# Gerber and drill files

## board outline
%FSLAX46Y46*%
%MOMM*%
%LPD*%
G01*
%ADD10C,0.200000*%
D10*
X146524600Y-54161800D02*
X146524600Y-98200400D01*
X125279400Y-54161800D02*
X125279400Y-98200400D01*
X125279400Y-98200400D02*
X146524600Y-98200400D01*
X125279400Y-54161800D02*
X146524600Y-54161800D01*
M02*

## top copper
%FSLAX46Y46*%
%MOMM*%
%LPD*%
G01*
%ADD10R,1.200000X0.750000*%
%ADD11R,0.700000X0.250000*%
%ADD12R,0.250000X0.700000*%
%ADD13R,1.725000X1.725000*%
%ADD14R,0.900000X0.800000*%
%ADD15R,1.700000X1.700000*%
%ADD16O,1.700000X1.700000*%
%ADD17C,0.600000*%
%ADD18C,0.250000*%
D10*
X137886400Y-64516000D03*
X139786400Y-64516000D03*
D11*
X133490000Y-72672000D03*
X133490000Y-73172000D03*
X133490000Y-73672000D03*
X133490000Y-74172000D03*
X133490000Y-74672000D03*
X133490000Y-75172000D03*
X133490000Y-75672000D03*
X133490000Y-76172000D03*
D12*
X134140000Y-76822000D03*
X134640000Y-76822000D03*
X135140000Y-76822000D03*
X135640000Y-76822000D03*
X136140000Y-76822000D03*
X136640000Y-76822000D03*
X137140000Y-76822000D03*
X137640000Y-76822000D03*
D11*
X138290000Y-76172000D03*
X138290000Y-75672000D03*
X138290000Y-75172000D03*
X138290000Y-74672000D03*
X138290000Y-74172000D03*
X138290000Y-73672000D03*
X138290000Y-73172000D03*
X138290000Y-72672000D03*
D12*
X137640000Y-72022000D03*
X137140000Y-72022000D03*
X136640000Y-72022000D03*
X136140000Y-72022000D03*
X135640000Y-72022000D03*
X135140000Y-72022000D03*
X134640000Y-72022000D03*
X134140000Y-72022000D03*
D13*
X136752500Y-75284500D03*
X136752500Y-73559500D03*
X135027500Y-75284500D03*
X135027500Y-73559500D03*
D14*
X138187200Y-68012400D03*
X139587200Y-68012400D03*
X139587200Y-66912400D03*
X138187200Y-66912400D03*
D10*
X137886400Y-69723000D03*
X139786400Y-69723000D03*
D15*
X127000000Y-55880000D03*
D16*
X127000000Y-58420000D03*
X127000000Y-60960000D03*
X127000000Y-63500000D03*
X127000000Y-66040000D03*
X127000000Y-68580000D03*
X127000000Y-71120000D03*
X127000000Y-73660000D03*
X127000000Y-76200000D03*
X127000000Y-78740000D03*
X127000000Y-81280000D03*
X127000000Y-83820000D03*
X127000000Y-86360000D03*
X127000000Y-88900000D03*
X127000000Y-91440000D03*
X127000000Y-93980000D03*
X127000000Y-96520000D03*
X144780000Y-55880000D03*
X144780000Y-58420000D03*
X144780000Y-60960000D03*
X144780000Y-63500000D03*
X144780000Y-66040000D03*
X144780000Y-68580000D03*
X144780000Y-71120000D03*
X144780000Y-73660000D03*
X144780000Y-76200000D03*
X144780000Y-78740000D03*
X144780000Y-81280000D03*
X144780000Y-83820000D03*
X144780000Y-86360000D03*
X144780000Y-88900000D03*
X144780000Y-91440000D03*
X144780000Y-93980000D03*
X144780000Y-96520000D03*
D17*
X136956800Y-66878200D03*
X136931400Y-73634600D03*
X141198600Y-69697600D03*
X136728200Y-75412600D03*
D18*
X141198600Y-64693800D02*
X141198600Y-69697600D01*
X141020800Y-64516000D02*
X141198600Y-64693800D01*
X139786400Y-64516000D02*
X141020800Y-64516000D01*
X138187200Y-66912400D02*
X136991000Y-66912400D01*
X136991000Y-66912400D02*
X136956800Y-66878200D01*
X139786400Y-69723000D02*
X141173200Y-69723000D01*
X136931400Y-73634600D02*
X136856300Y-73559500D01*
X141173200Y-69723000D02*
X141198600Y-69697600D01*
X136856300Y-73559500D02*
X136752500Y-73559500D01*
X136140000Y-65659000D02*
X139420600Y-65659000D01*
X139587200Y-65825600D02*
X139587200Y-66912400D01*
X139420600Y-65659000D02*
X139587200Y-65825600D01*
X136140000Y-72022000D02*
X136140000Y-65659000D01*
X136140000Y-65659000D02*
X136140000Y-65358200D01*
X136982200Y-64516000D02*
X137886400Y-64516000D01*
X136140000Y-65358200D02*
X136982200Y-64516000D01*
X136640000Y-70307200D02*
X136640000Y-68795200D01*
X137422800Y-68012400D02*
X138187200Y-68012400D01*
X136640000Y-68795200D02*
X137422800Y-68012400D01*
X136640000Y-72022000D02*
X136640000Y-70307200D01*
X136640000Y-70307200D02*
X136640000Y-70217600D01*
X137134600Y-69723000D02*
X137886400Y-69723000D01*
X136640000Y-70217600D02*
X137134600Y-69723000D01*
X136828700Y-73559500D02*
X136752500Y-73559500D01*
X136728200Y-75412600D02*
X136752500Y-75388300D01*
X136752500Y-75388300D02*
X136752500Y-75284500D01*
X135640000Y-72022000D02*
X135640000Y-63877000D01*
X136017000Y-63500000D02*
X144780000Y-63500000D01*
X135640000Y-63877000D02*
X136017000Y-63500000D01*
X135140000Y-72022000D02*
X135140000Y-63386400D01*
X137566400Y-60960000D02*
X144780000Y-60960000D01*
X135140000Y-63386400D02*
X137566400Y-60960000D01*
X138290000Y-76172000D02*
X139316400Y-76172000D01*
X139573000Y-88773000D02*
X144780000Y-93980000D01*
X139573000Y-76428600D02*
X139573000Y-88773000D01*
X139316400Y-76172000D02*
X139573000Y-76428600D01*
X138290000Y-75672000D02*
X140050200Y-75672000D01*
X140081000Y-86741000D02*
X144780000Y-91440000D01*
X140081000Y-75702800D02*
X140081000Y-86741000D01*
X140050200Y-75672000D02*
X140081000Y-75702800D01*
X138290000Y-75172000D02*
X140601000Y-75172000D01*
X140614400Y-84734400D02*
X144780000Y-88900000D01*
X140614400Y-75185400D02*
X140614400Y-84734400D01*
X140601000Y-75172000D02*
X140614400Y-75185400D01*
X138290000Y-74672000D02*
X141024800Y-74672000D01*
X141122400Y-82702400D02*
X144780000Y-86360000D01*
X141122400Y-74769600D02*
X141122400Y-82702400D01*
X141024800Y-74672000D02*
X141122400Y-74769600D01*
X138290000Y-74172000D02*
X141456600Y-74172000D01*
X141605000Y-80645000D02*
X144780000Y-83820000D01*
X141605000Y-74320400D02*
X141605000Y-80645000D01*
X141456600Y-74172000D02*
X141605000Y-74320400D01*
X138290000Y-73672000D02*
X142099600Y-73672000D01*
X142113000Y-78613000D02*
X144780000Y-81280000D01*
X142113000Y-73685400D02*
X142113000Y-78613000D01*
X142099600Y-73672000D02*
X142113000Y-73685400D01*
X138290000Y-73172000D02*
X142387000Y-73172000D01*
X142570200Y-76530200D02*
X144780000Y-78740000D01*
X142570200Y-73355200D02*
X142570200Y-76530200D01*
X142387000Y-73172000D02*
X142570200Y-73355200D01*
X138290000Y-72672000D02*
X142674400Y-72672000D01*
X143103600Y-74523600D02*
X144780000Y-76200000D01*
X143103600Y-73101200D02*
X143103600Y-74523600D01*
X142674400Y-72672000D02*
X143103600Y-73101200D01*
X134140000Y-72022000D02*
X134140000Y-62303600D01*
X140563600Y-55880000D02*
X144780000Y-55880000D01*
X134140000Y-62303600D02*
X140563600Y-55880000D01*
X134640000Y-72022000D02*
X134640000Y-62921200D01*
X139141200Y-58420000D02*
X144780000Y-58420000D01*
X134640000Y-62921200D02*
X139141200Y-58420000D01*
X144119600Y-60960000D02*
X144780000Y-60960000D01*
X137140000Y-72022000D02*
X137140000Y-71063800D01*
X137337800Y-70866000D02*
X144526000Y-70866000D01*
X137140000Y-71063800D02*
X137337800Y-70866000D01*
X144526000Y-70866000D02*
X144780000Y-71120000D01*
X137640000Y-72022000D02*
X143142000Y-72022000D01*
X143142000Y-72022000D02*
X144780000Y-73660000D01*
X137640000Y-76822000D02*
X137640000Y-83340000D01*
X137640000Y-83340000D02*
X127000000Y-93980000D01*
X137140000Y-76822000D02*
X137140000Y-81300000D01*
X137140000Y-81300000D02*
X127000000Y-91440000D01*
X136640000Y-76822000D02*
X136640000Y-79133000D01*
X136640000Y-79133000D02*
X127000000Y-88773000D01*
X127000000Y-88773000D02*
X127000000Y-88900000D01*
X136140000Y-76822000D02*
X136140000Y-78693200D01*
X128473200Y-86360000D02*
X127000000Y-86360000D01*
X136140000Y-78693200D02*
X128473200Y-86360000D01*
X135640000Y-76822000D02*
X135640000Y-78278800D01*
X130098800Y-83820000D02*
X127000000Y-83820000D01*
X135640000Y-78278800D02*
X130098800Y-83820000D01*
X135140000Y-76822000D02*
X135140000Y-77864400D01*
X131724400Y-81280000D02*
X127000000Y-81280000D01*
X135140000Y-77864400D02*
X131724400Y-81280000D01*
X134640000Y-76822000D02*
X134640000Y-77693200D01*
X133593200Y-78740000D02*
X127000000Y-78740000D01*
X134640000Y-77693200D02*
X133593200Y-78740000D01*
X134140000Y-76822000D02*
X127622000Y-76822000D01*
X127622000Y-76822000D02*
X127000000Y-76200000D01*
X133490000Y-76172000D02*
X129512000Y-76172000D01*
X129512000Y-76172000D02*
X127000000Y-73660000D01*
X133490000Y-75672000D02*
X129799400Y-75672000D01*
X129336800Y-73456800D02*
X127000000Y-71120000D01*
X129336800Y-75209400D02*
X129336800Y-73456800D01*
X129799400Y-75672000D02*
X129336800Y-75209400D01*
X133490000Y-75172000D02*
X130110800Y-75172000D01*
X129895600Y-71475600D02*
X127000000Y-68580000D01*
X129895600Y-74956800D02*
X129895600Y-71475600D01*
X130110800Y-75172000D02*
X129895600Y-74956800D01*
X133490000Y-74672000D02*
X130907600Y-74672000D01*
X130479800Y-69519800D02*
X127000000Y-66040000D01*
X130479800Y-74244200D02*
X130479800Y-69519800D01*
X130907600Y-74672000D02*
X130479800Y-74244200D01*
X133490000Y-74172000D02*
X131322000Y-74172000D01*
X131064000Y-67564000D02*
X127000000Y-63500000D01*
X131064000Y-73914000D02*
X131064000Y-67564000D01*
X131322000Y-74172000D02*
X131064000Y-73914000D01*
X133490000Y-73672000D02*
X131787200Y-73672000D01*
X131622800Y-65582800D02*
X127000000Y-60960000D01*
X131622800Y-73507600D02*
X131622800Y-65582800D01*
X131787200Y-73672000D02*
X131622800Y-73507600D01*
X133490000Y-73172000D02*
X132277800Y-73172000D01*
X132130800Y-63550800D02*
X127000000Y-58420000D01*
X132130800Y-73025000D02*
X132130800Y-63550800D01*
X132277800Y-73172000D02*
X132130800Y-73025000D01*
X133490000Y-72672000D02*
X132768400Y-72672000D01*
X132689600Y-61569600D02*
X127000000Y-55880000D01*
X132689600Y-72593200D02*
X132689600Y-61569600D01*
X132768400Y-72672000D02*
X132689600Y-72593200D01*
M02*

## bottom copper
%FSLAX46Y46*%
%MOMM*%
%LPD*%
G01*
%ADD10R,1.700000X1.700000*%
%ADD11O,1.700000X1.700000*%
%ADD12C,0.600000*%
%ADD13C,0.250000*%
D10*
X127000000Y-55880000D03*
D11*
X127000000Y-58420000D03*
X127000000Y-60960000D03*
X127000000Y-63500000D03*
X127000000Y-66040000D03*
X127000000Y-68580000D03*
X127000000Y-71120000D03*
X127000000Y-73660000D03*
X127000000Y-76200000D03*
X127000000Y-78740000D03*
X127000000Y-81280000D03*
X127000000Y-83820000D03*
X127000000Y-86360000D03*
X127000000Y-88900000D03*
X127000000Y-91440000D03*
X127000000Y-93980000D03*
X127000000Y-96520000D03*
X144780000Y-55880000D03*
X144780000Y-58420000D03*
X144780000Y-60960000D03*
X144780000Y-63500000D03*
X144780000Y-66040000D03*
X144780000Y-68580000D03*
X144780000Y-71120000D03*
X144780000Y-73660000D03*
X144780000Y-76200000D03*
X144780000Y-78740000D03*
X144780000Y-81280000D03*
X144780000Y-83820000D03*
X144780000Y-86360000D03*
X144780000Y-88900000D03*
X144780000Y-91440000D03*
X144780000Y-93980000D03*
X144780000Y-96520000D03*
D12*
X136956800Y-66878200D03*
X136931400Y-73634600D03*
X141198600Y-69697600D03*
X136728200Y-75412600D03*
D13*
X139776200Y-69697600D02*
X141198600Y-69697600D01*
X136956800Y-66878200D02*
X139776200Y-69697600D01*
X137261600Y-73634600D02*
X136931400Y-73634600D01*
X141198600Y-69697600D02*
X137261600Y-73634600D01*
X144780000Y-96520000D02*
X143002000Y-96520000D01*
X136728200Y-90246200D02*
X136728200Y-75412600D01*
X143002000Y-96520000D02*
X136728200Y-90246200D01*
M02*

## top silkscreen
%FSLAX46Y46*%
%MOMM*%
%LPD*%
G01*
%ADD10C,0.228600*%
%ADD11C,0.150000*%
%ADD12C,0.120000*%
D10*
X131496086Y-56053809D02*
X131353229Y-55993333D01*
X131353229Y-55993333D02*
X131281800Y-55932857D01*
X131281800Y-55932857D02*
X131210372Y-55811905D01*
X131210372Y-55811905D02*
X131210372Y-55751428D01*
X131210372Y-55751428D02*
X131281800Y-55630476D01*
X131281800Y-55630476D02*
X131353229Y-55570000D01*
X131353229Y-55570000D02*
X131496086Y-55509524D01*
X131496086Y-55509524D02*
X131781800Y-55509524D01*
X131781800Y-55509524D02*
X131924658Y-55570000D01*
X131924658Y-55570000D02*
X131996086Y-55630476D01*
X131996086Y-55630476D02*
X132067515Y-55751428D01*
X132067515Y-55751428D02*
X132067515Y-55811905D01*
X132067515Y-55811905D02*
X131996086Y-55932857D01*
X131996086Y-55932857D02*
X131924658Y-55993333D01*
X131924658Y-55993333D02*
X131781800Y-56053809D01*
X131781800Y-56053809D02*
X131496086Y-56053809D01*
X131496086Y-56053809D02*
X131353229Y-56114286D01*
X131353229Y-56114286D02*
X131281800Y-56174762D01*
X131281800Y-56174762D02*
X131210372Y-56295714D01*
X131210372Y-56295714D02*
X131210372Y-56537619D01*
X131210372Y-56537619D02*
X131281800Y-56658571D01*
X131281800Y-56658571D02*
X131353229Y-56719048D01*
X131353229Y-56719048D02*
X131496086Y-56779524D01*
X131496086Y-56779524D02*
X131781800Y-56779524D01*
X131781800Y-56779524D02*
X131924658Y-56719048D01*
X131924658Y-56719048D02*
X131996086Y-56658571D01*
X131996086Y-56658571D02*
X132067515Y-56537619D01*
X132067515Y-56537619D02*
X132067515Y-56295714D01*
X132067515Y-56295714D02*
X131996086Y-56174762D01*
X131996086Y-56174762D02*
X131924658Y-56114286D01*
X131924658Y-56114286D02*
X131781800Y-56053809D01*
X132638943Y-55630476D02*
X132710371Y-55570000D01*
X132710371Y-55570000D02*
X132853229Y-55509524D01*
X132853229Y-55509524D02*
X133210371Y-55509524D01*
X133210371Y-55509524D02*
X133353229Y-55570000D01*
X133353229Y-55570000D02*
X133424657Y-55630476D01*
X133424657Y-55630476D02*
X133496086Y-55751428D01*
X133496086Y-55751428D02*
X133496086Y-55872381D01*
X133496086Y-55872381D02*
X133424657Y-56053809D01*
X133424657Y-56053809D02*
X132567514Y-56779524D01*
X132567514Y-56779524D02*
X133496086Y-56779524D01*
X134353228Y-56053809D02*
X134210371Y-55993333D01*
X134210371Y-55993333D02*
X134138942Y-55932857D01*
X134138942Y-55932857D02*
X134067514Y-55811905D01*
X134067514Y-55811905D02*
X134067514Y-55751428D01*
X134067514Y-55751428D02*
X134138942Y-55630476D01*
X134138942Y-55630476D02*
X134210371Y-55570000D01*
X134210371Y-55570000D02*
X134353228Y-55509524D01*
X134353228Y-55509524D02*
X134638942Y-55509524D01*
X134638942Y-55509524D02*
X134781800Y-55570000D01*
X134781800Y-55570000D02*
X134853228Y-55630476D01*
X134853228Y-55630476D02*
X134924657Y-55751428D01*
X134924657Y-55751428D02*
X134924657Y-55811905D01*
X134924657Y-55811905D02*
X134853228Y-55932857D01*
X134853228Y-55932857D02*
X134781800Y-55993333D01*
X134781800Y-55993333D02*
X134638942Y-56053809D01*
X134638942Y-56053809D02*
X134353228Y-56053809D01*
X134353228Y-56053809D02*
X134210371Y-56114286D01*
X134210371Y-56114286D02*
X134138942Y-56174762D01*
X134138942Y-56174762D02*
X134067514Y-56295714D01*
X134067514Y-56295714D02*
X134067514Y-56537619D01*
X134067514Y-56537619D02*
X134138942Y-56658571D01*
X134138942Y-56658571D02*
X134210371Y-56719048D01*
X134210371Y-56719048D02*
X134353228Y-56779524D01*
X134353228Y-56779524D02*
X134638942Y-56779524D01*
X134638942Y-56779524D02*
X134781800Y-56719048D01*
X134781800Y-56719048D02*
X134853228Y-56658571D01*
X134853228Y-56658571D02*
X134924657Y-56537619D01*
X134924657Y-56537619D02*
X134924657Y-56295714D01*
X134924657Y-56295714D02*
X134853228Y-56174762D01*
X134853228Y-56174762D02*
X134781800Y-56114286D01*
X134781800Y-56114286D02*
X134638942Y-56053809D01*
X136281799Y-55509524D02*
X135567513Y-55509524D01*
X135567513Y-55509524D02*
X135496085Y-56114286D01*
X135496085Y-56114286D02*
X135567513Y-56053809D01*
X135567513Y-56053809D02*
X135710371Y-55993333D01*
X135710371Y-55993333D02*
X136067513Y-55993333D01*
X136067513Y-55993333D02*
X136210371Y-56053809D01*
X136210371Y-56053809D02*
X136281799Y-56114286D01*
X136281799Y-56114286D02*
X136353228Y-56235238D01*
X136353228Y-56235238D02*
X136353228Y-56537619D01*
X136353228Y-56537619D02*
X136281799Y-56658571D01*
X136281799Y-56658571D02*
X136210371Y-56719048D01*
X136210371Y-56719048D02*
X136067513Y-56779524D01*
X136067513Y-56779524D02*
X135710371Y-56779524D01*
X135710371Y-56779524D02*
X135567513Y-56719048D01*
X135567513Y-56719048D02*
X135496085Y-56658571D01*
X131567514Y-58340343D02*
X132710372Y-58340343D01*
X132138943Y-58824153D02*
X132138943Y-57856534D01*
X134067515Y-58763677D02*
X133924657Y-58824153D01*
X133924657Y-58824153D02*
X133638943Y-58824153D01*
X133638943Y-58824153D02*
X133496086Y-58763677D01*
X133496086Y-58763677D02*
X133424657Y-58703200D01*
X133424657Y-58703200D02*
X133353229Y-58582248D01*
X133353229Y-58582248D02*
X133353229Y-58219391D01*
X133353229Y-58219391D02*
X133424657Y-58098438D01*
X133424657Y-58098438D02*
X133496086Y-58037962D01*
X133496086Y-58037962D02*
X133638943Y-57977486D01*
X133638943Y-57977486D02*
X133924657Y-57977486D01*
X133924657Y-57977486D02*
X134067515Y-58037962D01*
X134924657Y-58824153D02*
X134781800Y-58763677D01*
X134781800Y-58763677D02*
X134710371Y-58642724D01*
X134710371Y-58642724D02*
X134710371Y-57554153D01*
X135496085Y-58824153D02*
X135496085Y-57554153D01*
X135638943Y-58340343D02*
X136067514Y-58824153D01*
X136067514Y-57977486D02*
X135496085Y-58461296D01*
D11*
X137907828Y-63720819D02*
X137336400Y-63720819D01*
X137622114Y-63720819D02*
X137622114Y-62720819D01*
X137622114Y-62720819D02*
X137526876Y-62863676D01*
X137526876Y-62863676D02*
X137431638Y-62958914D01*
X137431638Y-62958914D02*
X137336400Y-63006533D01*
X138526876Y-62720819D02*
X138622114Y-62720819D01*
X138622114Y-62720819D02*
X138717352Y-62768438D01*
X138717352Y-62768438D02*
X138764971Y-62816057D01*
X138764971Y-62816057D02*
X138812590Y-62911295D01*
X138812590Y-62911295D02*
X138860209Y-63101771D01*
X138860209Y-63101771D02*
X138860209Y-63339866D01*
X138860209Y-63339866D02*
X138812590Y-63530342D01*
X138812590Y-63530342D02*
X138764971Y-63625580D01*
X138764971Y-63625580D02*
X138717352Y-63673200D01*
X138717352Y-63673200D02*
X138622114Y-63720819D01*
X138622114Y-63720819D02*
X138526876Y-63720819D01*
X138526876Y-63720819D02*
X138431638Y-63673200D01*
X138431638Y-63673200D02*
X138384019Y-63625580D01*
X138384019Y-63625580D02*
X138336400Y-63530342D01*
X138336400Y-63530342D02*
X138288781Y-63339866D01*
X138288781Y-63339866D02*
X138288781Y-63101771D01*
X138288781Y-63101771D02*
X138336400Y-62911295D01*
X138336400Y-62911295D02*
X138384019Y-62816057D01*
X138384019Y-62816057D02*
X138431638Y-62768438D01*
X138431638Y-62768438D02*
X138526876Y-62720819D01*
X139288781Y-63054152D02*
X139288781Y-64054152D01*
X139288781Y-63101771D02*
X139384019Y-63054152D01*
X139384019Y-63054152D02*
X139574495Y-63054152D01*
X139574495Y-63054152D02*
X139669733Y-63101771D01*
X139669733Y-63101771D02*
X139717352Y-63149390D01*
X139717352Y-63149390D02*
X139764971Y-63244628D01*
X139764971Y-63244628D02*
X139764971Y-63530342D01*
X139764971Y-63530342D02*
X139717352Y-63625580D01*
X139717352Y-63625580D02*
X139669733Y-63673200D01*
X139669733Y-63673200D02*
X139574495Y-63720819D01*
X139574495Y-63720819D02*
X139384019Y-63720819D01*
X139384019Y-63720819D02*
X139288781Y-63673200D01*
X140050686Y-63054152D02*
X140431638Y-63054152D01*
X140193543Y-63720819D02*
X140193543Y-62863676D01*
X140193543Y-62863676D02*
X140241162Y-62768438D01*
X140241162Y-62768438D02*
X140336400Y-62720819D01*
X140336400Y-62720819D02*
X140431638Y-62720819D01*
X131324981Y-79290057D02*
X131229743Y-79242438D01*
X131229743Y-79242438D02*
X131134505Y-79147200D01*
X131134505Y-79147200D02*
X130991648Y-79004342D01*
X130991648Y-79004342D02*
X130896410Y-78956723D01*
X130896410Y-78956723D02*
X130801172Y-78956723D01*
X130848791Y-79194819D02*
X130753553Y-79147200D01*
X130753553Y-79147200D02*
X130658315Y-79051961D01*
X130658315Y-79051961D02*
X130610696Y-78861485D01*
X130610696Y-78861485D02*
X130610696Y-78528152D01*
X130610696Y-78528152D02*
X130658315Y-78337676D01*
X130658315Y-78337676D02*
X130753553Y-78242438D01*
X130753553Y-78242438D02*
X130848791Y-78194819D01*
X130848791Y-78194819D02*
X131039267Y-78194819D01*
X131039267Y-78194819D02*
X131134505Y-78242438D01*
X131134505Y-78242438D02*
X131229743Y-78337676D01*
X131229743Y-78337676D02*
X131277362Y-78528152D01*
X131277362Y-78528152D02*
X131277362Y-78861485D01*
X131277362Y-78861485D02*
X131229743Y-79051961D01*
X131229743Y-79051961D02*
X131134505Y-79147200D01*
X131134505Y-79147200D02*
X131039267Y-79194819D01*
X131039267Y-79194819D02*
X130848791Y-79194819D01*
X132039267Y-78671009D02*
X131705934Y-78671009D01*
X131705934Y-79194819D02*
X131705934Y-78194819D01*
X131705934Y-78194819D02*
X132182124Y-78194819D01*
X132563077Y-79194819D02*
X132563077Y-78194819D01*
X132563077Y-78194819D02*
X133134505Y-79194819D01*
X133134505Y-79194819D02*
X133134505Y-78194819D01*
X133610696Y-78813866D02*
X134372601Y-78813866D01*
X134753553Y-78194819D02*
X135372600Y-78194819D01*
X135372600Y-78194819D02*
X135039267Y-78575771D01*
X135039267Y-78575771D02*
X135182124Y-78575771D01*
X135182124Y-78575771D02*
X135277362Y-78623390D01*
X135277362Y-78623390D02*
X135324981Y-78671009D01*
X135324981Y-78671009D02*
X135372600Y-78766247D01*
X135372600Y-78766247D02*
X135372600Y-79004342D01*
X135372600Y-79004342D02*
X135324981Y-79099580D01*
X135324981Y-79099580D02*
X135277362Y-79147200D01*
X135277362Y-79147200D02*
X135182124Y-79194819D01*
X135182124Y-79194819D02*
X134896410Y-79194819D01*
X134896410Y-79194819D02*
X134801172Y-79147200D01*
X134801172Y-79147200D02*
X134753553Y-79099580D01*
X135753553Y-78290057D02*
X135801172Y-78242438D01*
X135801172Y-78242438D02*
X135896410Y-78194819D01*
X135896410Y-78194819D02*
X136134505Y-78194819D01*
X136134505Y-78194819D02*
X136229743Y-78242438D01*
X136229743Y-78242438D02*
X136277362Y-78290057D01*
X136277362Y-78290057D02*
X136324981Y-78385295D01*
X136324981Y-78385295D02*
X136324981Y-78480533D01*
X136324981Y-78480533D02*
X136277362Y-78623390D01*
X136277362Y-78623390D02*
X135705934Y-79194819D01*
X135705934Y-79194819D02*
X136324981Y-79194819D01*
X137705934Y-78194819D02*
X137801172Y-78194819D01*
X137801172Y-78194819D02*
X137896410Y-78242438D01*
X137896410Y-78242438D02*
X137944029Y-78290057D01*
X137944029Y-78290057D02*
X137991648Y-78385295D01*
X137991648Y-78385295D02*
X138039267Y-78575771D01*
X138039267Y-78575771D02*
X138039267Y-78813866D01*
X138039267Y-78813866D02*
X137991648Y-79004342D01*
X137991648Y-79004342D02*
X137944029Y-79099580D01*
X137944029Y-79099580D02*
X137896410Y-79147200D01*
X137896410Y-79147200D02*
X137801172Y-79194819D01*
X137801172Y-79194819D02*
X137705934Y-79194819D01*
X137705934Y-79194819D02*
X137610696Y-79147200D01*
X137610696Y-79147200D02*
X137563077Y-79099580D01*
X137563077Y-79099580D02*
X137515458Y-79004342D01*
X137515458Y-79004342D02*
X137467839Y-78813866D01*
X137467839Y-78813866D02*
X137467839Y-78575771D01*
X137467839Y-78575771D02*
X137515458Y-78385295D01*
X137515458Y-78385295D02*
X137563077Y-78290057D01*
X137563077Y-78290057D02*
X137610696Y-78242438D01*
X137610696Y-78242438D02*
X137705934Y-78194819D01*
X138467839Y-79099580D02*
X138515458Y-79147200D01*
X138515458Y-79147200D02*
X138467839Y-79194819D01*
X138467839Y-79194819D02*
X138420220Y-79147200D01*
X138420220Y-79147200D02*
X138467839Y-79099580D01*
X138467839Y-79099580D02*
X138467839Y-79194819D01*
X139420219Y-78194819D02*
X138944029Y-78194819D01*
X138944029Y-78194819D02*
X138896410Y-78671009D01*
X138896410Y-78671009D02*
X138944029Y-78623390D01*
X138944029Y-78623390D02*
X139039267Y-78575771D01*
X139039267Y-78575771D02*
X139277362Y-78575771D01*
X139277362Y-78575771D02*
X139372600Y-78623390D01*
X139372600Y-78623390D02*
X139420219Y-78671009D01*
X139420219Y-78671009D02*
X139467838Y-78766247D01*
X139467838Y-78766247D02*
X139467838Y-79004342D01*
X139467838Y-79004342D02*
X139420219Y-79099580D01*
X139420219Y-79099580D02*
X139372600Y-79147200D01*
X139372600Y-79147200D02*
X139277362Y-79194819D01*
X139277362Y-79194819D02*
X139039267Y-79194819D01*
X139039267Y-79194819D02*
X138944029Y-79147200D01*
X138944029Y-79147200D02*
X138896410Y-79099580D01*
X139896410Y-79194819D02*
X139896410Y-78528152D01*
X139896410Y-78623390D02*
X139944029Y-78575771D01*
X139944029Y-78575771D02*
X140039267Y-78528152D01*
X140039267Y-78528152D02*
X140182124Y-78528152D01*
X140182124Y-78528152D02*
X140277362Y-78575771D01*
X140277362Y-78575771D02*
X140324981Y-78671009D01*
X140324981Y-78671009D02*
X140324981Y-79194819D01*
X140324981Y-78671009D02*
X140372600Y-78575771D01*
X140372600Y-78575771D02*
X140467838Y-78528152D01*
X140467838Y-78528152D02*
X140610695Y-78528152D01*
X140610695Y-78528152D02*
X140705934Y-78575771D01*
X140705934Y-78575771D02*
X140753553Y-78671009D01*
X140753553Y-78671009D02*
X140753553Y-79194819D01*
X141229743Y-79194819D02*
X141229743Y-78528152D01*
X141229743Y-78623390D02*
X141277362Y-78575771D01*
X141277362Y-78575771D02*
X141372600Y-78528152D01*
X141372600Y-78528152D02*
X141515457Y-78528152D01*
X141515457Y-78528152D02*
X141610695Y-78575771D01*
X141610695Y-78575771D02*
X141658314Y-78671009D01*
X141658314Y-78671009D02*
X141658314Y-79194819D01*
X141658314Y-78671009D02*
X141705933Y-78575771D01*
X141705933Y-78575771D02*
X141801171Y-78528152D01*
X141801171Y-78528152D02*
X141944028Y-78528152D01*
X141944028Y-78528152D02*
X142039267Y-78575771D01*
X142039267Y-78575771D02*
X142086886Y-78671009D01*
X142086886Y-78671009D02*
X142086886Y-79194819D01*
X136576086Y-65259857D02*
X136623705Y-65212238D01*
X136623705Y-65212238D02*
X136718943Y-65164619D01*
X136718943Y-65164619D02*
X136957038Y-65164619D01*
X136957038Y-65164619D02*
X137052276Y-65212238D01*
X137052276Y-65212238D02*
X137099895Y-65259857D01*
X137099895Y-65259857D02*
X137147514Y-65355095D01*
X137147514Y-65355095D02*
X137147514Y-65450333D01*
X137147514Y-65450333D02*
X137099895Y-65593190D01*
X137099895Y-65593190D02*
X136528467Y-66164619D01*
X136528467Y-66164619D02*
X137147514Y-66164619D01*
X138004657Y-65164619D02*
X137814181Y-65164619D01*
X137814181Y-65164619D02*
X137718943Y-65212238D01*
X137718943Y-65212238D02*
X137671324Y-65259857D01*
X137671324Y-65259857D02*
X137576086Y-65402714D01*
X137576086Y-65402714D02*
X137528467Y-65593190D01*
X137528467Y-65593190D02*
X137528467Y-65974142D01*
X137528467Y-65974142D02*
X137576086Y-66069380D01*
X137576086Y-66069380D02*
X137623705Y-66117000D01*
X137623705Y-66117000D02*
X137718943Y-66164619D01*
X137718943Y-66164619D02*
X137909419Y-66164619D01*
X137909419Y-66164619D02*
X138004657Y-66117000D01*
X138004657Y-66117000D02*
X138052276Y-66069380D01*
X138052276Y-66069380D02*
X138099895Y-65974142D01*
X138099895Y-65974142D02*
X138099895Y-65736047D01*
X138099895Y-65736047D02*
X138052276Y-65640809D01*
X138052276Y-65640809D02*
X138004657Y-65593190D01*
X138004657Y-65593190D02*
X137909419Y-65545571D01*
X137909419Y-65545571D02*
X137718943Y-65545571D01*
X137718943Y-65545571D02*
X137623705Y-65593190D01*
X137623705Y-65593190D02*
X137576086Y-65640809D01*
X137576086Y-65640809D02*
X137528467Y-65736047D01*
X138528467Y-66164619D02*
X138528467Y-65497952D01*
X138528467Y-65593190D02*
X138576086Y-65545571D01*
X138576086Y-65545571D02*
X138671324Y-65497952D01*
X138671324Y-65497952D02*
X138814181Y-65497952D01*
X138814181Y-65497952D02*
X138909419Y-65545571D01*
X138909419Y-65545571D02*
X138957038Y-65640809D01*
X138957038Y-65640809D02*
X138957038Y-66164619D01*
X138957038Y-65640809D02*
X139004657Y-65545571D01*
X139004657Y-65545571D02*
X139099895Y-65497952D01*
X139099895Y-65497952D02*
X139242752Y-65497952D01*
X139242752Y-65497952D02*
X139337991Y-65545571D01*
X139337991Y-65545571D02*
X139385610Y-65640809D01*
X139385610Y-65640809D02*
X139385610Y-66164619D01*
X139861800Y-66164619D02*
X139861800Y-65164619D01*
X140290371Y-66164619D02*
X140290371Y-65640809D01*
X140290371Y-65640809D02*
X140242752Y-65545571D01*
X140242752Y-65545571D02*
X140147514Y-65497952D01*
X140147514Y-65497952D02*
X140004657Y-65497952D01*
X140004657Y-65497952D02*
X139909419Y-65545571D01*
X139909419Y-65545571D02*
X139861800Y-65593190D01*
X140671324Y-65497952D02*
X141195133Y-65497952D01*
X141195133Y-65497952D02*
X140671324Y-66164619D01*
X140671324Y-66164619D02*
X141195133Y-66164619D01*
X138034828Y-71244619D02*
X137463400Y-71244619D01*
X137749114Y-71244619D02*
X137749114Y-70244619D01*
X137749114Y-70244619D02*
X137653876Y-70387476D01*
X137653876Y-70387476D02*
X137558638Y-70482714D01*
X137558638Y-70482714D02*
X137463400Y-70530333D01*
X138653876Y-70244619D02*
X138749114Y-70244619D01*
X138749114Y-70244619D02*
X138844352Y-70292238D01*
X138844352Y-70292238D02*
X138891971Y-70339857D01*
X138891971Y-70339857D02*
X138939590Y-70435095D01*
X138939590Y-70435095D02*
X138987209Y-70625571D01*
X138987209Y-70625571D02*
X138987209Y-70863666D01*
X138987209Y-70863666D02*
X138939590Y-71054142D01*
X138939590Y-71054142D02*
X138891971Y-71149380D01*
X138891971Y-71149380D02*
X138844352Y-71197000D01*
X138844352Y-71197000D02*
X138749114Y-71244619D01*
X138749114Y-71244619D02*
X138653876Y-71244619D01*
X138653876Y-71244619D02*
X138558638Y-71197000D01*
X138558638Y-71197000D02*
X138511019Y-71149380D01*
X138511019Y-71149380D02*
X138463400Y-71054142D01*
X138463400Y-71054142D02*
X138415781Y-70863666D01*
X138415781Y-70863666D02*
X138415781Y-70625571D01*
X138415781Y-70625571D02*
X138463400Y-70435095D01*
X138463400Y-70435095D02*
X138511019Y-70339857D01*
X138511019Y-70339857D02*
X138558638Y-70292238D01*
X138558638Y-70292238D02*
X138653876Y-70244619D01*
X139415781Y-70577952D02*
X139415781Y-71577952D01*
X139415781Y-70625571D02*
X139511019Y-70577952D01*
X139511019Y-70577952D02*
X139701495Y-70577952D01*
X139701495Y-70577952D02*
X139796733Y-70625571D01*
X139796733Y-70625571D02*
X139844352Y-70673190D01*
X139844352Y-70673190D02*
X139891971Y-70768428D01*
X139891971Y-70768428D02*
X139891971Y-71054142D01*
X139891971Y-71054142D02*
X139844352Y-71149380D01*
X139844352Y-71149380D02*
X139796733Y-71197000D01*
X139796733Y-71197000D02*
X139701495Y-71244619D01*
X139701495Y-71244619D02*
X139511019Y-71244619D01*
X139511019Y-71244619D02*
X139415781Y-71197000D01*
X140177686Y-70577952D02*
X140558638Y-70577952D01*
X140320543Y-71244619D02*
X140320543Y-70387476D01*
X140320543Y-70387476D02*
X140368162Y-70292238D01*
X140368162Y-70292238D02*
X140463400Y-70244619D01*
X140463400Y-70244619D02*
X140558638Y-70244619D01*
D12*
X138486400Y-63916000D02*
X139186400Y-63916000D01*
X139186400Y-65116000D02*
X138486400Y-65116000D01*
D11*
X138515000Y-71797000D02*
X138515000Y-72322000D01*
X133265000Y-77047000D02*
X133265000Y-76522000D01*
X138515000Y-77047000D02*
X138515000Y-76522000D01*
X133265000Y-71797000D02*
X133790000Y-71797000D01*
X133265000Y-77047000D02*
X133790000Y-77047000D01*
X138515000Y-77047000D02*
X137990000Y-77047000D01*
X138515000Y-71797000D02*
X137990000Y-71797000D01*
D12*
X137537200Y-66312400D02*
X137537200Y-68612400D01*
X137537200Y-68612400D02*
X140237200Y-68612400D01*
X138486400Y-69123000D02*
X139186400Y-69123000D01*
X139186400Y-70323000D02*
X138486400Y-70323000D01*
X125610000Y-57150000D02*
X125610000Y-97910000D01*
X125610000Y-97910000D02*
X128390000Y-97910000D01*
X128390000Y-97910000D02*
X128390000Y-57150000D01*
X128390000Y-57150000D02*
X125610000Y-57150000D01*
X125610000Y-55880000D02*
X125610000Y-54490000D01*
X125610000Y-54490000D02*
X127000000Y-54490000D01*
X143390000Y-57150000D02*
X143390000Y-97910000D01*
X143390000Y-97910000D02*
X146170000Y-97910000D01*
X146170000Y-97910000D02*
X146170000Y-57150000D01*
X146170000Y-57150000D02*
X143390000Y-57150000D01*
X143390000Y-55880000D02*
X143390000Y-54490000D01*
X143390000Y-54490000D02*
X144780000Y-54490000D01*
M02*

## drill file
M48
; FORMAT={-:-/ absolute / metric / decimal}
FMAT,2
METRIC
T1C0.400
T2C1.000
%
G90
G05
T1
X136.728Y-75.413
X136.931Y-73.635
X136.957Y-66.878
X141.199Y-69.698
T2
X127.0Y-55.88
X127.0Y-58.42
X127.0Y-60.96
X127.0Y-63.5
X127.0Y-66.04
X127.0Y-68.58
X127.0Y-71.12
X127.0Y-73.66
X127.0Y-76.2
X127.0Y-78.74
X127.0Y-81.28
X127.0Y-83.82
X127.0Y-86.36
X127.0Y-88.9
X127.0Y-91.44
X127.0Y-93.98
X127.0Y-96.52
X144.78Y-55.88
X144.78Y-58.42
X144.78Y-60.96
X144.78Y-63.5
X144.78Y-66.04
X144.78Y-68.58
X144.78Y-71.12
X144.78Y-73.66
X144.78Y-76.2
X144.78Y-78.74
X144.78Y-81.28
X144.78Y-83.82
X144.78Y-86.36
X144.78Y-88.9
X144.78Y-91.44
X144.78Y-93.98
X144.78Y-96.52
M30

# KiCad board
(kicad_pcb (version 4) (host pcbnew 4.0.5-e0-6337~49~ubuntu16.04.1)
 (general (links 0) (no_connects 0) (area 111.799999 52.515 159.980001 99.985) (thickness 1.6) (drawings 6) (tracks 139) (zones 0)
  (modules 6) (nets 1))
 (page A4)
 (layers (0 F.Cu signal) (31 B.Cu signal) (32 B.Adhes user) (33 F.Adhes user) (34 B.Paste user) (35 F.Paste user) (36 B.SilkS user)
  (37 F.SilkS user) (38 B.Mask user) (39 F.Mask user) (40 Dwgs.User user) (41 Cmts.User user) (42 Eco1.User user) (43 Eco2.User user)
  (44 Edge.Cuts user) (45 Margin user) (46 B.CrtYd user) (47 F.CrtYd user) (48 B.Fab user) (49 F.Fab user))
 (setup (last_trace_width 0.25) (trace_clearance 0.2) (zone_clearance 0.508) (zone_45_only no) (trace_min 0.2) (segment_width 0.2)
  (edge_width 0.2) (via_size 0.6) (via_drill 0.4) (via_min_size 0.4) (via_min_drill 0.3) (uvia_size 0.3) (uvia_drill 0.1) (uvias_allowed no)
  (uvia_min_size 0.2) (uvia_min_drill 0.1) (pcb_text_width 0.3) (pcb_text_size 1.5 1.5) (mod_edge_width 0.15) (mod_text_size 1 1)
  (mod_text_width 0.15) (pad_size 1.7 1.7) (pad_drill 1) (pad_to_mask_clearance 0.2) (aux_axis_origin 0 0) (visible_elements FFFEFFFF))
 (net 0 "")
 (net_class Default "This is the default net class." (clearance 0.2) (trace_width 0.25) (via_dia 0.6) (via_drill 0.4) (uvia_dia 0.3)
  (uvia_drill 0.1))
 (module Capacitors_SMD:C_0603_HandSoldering (layer F.Cu) (at 138.8364 64.516)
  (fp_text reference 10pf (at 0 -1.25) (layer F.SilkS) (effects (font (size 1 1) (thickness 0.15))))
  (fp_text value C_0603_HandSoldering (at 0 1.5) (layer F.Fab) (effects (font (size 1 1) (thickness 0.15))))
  (fp_line (start -0.35 -0.6) (end 0.35 -0.6) (layer F.SilkS) (width 0.12))
  (fp_line (start 0.35 0.6) (end -0.35 0.6) (layer F.SilkS) (width 0.12))
  (pad 1 smd rect (at -0.95 0) (size 1.2 0.75) (layers F.Cu F.Paste F.Mask))
  (pad 2 smd rect (at 0.95 0) (size 1.2 0.75) (layers F.Cu F.Paste F.Mask)))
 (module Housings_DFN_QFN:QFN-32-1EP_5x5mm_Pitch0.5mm (layer F.Cu) (at 135.89 74.422)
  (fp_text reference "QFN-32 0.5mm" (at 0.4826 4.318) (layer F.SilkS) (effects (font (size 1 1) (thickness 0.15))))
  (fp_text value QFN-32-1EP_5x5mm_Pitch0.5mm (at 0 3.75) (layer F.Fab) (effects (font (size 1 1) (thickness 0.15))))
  (fp_line (start 2.625 -2.625) (end 2.625 -2.1) (layer F.SilkS) (width 0.15))
  (fp_line (start -2.625 2.625) (end -2.625 2.1) (layer F.SilkS) (width 0.15))
  (fp_line (start 2.625 2.625) (end 2.625 2.1) (layer F.SilkS) (width 0.15))
  (fp_line (start -2.625 -2.625) (end -2.1 -2.625) (layer F.SilkS) (width 0.15))
  (fp_line (start -2.625 2.625) (end -2.1 2.625) (layer F.SilkS) (width 0.15))
  (fp_line (start 2.625 2.625) (end 2.1 2.625) (layer F.SilkS) (width 0.15))
  (fp_line (start 2.625 -2.625) (end 2.1 -2.625) (layer F.SilkS) (width 0.15))
  (pad 1 smd rect (at -2.4 -1.75) (size 0.7 0.25) (layers F.Cu F.Paste F.Mask))
  (pad 2 smd rect (at -2.4 -1.25) (size 0.7 0.25) (layers F.Cu F.Paste F.Mask))
  (pad 3 smd rect (at -2.4 -0.75) (size 0.7 0.25) (layers F.Cu F.Paste F.Mask))
  (pad 4 smd rect (at -2.4 -0.25) (size 0.7 0.25) (layers F.Cu F.Paste F.Mask))
  (pad 5 smd rect (at -2.4 0.25) (size 0.7 0.25) (layers F.Cu F.Paste F.Mask))
  (pad 6 smd rect (at -2.4 0.75) (size 0.7 0.25) (layers F.Cu F.Paste F.Mask))
  (pad 7 smd rect (at -2.4 1.25) (size 0.7 0.25) (layers F.Cu F.Paste F.Mask))
  (pad 8 smd rect (at -2.4 1.75) (size 0.7 0.25) (layers F.Cu F.Paste F.Mask))
  (pad 9 smd rect (at -1.75 2.4 90) (size 0.7 0.25) (layers F.Cu F.Paste F.Mask))
  (pad 10 smd rect (at -1.25 2.4 90) (size 0.7 0.25) (layers F.Cu F.Paste F.Mask))
  (pad 11 smd rect (at -0.75 2.4 90) (size 0.7 0.25) (layers F.Cu F.Paste F.Mask))
  (pad 12 smd rect (at -0.25 2.4 90) (size 0.7 0.25) (layers F.Cu F.Paste F.Mask))
  (pad 13 smd rect (at 0.25 2.4 90) (size 0.7 0.25) (layers F.Cu F.Paste F.Mask))
  (pad 14 smd rect (at 0.75 2.4 90) (size 0.7 0.25) (layers F.Cu F.Paste F.Mask))
  (pad 15 smd rect (at 1.25 2.4 90) (size 0.7 0.25) (layers F.Cu F.Paste F.Mask))
  (pad 16 smd rect (at 1.75 2.4 90) (size 0.7 0.25) (layers F.Cu F.Paste F.Mask))
  (pad 17 smd rect (at 2.4 1.75) (size 0.7 0.25) (layers F.Cu F.Paste F.Mask))
  (pad 18 smd rect (at 2.4 1.25) (size 0.7 0.25) (layers F.Cu F.Paste F.Mask))
  (pad 19 smd rect (at 2.4 0.75) (size 0.7 0.25) (layers F.Cu F.Paste F.Mask))
  (pad 20 smd rect (at 2.4 0.25) (size 0.7 0.25) (layers F.Cu F.Paste F.Mask))
  (pad 21 smd rect (at 2.4 -0.25) (size 0.7 0.25) (layers F.Cu F.Paste F.Mask))
  (pad 22 smd rect (at 2.4 -0.75) (size 0.7 0.25) (layers F.Cu F.Paste F.Mask))
  (pad 23 smd rect (at 2.4 -1.25) (size 0.7 0.25) (layers F.Cu F.Paste F.Mask))
  (pad 24 smd rect (at 2.4 -1.75) (size 0.7 0.25) (layers F.Cu F.Paste F.Mask))
  (pad 25 smd rect (at 1.75 -2.4 90) (size 0.7 0.25) (layers F.Cu F.Paste F.Mask))
  (pad 26 smd rect (at 1.25 -2.4 90) (size 0.7 0.25) (layers F.Cu F.Paste F.Mask))
  (pad 27 smd rect (at 0.75 -2.4 90) (size 0.7 0.25) (layers F.Cu F.Paste F.Mask))
  (pad 28 smd rect (at 0.25 -2.4 90) (size 0.7 0.25) (layers F.Cu F.Paste F.Mask))
  (pad 29 smd rect (at -0.25 -2.4 90) (size 0.7 0.25) (layers F.Cu F.Paste F.Mask))
  (pad 30 smd rect (at -0.75 -2.4 90) (size 0.7 0.25) (layers F.Cu F.Paste F.Mask))
  (pad 31 smd rect (at -1.25 -2.4 90) (size 0.7 0.25) (layers F.Cu F.Paste F.Mask))
  (pad 32 smd rect (at -1.75 -2.4 90) (size 0.7 0.25) (layers F.Cu F.Paste F.Mask))
  (pad 33 smd rect (at 0.8625 0.8625) (size 1.725 1.725) (layers F.Cu F.Paste F.Mask) (solder_paste_margin_ratio -0.2))
  (pad 33 smd rect (at 0.8625 -0.8625) (size 1.725 1.725) (layers F.Cu F.Paste F.Mask) (solder_paste_margin_ratio -0.2))
  (pad 33 smd rect (at -0.8625 0.8625) (size 1.725 1.725) (layers F.Cu F.Paste F.Mask) (solder_paste_margin_ratio -0.2))
  (pad 33 smd rect (at -0.8625 -0.8625) (size 1.725 1.725) (layers F.Cu F.Paste F.Mask) (solder_paste_margin_ratio -0.2)))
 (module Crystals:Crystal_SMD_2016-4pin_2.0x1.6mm (layer F.Cu) (at 138.8872 67.4624)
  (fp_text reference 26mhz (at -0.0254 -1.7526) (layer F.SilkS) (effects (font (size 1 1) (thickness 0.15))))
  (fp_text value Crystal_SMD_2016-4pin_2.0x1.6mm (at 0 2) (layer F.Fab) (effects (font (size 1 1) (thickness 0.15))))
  (fp_line (start -1.35 -1.15) (end -1.35 1.15) (layer F.SilkS) (width 0.12))
  (fp_line (start -1.35 1.15) (end 1.35 1.15) (layer F.SilkS) (width 0.12))
  (pad 1 smd rect (at -0.7 0.55) (size 0.9 0.8) (layers F.Cu F.Mask))
  (pad 2 smd rect (at 0.7 0.55) (size 0.9 0.8) (layers F.Cu F.Mask))
  (pad 3 smd rect (at 0.7 -0.55) (size 0.9 0.8) (layers F.Cu F.Mask))
  (pad 4 smd rect (at -0.7 -0.55) (size 0.9 0.8) (layers F.Cu F.Mask)))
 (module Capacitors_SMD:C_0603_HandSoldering (layer F.Cu) (at 138.8364 69.723)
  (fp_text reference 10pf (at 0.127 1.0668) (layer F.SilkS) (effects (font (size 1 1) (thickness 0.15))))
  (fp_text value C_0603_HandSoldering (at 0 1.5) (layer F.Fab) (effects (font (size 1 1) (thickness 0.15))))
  (fp_line (start -0.35 -0.6) (end 0.35 -0.6) (layer F.SilkS) (width 0.12))
  (fp_line (start 0.35 0.6) (end -0.35 0.6) (layer F.SilkS) (width 0.12))
  (pad 1 smd rect (at -0.95 0) (size 1.2 0.75) (layers F.Cu F.Paste F.Mask))
  (pad 2 smd rect (at 0.95 0) (size 1.2 0.75) (layers F.Cu F.Paste F.Mask)))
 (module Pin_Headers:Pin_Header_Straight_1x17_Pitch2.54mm (layer F.Cu) (at 127 55.88)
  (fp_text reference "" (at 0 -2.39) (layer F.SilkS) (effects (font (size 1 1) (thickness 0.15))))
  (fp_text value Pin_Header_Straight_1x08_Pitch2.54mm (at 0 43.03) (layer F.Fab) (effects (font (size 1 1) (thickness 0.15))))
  (fp_line (start -1.39 1.27) (end -1.39 42.03) (layer F.SilkS) (width 0.12))
  (fp_line (start -1.39 42.03) (end 1.39 42.03) (layer F.SilkS) (width 0.12))
  (fp_line (start 1.39 42.03) (end 1.39 1.27) (layer F.SilkS) (width 0.12))
  (fp_line (start 1.39 1.27) (end -1.39 1.27) (layer F.SilkS) (width 0.12))
  (fp_line (start -1.39 0) (end -1.39 -1.39) (layer F.SilkS) (width 0.12))
  (fp_line (start -1.39 -1.39) (end 0 -1.39) (layer F.SilkS) (width 0.12))
  (pad 1 thru_hole rect (at 0 0) (size 1.7 1.7) (drill 1) (layers *.Cu *.Mask))
  (pad 2 thru_hole oval (at 0 2.54) (size 1.7 1.7) (drill 1) (layers *.Cu *.Mask))
  (pad 3 thru_hole oval (at 0 5.08) (size 1.7 1.7) (drill 1) (layers *.Cu *.Mask))
  (pad 4 thru_hole oval (at 0 7.62) (size 1.7 1.7) (drill 1) (layers *.Cu *.Mask))
  (pad 5 thru_hole oval (at 0 10.16) (size 1.7 1.7) (drill 1) (layers *.Cu *.Mask))
  (pad 6 thru_hole oval (at 0 12.7) (size 1.7 1.7) (drill 1) (layers *.Cu *.Mask))
  (pad 7 thru_hole oval (at 0 15.24) (size 1.7 1.7) (drill 1) (layers *.Cu *.Mask))
  (pad 8 thru_hole oval (at 0 17.78) (size 1.7 1.7) (drill 1) (layers *.Cu *.Mask))
  (pad 9 thru_hole oval (at 0 20.32) (size 1.7 1.7) (drill 1) (layers *.Cu *.Mask))
  (pad 10 thru_hole oval (at 0 22.86) (size 1.7 1.7) (drill 1) (layers *.Cu *.Mask))
  (pad 11 thru_hole oval (at 0 25.4) (size 1.7 1.7) (drill 1) (layers *.Cu *.Mask))
  (pad 12 thru_hole oval (at 0 27.94) (size 1.7 1.7) (drill 1) (layers *.Cu *.Mask))
  (pad 13 thru_hole oval (at 0 30.48) (size 1.7 1.7) (drill 1) (layers *.Cu *.Mask))
  (pad 14 thru_hole oval (at 0 33.02) (size 1.7 1.7) (drill 1) (layers *.Cu *.Mask))
  (pad 15 thru_hole oval (at 0 35.56) (size 1.7 1.7) (drill 1) (layers *.Cu *.Mask))
  (pad 16 thru_hole oval (at 0 38.1) (size 1.7 1.7) (drill 1) (layers *.Cu *.Mask))
  (pad GND thru_hole oval (at 0 40.64) (size 1.7 1.7) (drill 1) (layers *.Cu *.Mask)))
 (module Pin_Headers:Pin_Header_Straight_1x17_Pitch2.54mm (layer F.Cu) (at 144.78 55.88)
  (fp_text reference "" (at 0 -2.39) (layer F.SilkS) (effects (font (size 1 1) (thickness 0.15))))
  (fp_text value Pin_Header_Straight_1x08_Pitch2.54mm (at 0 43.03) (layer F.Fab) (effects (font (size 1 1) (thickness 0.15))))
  (fp_line (start -1.39 1.27) (end -1.39 42.03) (layer F.SilkS) (width 0.12))
  (fp_line (start -1.39 42.03) (end 1.39 42.03) (layer F.SilkS) (width 0.12))
  (fp_line (start 1.39 42.03) (end 1.39 1.27) (layer F.SilkS) (width 0.12))
  (fp_line (start 1.39 1.27) (end -1.39 1.27) (layer F.SilkS) (width 0.12))
  (fp_line (start -1.39 0) (end -1.39 -1.39) (layer F.SilkS) (width 0.12))
  (fp_line (start -1.39 -1.39) (end 0 -1.39) (layer F.SilkS) (width 0.12))
  (pad 1 thru_hole oval (at 0 0) (size 1.7 1.7) (drill 1) (layers *.Cu *.Mask))
  (pad 2 thru_hole oval (at 0 2.54) (size 1.7 1.7) (drill 1) (layers *.Cu *.Mask))
  (pad 3 thru_hole oval (at 0 5.08) (size 1.7 1.7) (drill 1) (layers *.Cu *.Mask))
  (pad 4 thru_hole oval (at 0 7.62) (size 1.7 1.7) (drill 1) (layers *.Cu *.Mask))
  (pad 5 thru_hole oval (at 0 10.16) (size 1.7 1.7) (drill 1) (layers *.Cu *.Mask))
  (pad 6 thru_hole oval (at 0 12.7) (size 1.7 1.7) (drill 1) (layers *.Cu *.Mask))
  (pad 7 thru_hole oval (at 0 15.24) (size 1.7 1.7) (drill 1) (layers *.Cu *.Mask))
  (pad 8 thru_hole oval (at 0 17.78) (size 1.7 1.7) (drill 1) (layers *.Cu *.Mask))
  (pad 9 thru_hole oval (at 0 20.32) (size 1.7 1.7) (drill 1) (layers *.Cu *.Mask))
  (pad 10 thru_hole oval (at 0 22.86) (size 1.7 1.7) (drill 1) (layers *.Cu *.Mask))
  (pad 11 thru_hole oval (at 0 25.4) (size 1.7 1.7) (drill 1) (layers *.Cu *.Mask))
  (pad 12 thru_hole oval (at 0 27.94) (size 1.7 1.7) (drill 1) (layers *.Cu *.Mask))
  (pad 13 thru_hole oval (at 0 30.48) (size 1.7 1.7) (drill 1) (layers *.Cu *.Mask))
  (pad 14 thru_hole oval (at 0 33.02) (size 1.7 1.7) (drill 1) (layers *.Cu *.Mask))
  (pad 15 thru_hole oval (at 0 35.56) (size 1.7 1.7) (drill 1) (layers *.Cu *.Mask))
  (pad 16 thru_hole oval (at 0 38.1) (size 1.7 1.7) (drill 1) (layers *.Cu *.Mask))
  (pad GND thru_hole oval (at 0 40.64) (size 1.7 1.7) (drill 1) (layers *.Cu *.Mask)))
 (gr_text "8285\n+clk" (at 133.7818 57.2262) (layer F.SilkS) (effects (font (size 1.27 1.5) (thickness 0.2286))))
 (gr_line (start 146.5246 54.1618) (end 146.5246 98.2004) (angle 90) (layer Edge.Cuts) (width 0.2))
 (gr_line (start 125.2794 54.1618) (end 125.2794 98.2004) (angle 90) (layer Edge.Cuts) (width 0.2))
 (gr_line (start 125.2794 98.2004) (end 146.5246 98.2004) (angle 90) (layer Edge.Cuts) (width 0.2))
 (gr_line (start 125.2794 54.1618) (end 146.5246 54.1618) (angle 90) (layer Edge.Cuts) (width 0.2))
 (segment (start 141.1986 64.6938) (end 141.1986 69.6976) (width 0.25) (layer F.Cu) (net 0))
 (segment (start 141.0208 64.516) (end 141.1986 64.6938) (width 0.25) (layer F.Cu) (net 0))
 (segment (start 139.7864 64.516) (end 141.0208 64.516) (width 0.25) (layer F.Cu) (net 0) (status 10))
 (segment (start 138.1872 66.9124) (end 136.991 66.9124) (width 0.25) (layer F.Cu) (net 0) (status 10))
 (segment (start 139.7762 69.6976) (end 141.1986 69.6976) (width 0.25) (layer B.Cu) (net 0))
 (segment (start 136.9568 66.8782) (end 139.7762 69.6976) (width 0.25) (layer B.Cu) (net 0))
 (via (at 136.9568 66.8782) (size 0.6) (drill 0.4) (layers F.Cu B.Cu) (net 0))
 (segment (start 136.991 66.9124) (end 136.9568 66.8782) (width 0.25) (layer F.Cu) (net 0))
 (segment (start 139.7864 69.723) (end 141.1732 69.723) (width 0.25) (layer F.Cu) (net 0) (status 10))
 (segment (start 136.9314 73.6346) (end 136.8563 73.5595) (width 0.25) (layer F.Cu) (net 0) (status 30))
 (via (at 136.9314 73.6346) (size 0.6) (drill 0.4) (layers F.Cu B.Cu) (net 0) (status 30))
 (segment (start 137.2616 73.6346) (end 136.9314 73.6346) (width 0.25) (layer B.Cu) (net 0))
 (segment (start 141.1986 69.6976) (end 137.2616 73.6346) (width 0.25) (layer B.Cu) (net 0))
 (via (at 141.1986 69.6976) (size 0.6) (drill 0.4) (layers F.Cu B.Cu) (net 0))
 (segment (start 141.1732 69.723) (end 141.1986 69.6976) (width 0.25) (layer F.Cu) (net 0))
 (segment (start 136.8563 73.5595) (end 136.7525 73.5595) (width 0.25) (layer F.Cu) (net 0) (status 30))
 (segment (start 136.14 65.659) (end 139.4206 65.659) (width 0.25) (layer F.Cu) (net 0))
 (segment (start 139.5872 65.8256) (end 139.5872 66.9124) (width 0.25) (layer F.Cu) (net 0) (status 20))
 (segment (start 139.4206 65.659) (end 139.5872 65.8256) (width 0.25) (layer F.Cu) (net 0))
 (segment (start 136.14 72.022) (end 136.14 65.659) (width 0.25) (layer F.Cu) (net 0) (status 10))
 (segment (start 136.14 65.659) (end 136.14 65.3582) (width 0.25) (layer F.Cu) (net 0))
 (segment (start 136.9822 64.516) (end 137.8864 64.516) (width 0.25) (layer F.Cu) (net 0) (status 20))
 (segment (start 136.14 65.3582) (end 136.9822 64.516) (width 0.25) (layer F.Cu) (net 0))
 (segment (start 136.64 70.3072) (end 136.64 68.7952) (width 0.25) (layer F.Cu) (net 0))
 (segment (start 137.4228 68.0124) (end 138.1872 68.0124) (width 0.25) (layer F.Cu) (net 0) (status 20))
 (segment (start 136.64 68.7952) (end 137.4228 68.0124) (width 0.25) (layer F.Cu) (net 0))
 (segment (start 136.64 72.022) (end 136.64 70.3072) (width 0.25) (layer F.Cu) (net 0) (status 10))
 (segment (start 136.64 70.3072) (end 136.64 70.2176) (width 0.25) (layer F.Cu) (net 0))
 (segment (start 137.1346 69.723) (end 137.8864 69.723) (width 0.25) (layer F.Cu) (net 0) (status 20))
 (segment (start 136.64 70.2176) (end 137.1346 69.723) (width 0.25) (layer F.Cu) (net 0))
 (segment (start 136.8287 73.5595) (end 136.7525 73.5595) (width 0.25) (layer F.Cu) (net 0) (status 30))
 (segment (start 144.78 96.52) (end 143.002 96.52) (width 0.25) (layer B.Cu) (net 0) (status 10))
 (segment (start 136.7282 75.4126) (end 136.7525 75.3883) (width 0.25) (layer F.Cu) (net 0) (status 30))
 (via (at 136.7282 75.4126) (size 0.6) (drill 0.4) (layers F.Cu B.Cu) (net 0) (status 30))
 (segment (start 136.7282 90.2462) (end 136.7282 75.4126) (width 0.25) (layer B.Cu) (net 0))
 (segment (start 143.002 96.52) (end 136.7282 90.2462) (width 0.25) (layer B.Cu) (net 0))
 (segment (start 136.7525 75.3883) (end 136.7525 75.2845) (width 0.25) (layer F.Cu) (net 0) (status 30))
 (segment (start 135.64 72.022) (end 135.64 63.877) (width 0.25) (layer F.Cu) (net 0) (status 10))
 (segment (start 136.017 63.5) (end 144.78 63.5) (width 0.25) (layer F.Cu) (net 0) (status 20))
 (segment (start 135.64 63.877) (end 136.017 63.5) (width 0.25) (layer F.Cu) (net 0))
 (segment (start 135.14 72.022) (end 135.14 63.3864) (width 0.25) (layer F.Cu) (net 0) (status 10))
 (segment (start 137.5664 60.96) (end 144.78 60.96) (width 0.25) (layer F.Cu) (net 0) (status 20))
 (segment (start 135.14 63.3864) (end 137.5664 60.96) (width 0.25) (layer F.Cu) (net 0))
 (segment (start 138.29 76.172) (end 139.3164 76.172) (width 0.25) (layer F.Cu) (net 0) (status 10))
 (segment (start 139.573 88.773) (end 144.78 93.98) (width 0.25) (layer F.Cu) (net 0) (status 20))
 (segment (start 139.573 76.4286) (end 139.573 88.773) (width 0.25) (layer F.Cu) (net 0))
 (segment (start 139.3164 76.172) (end 139.573 76.4286) (width 0.25) (layer F.Cu) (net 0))
 (segment (start 138.29 75.672) (end 140.0502 75.672) (width 0.25) (layer F.Cu) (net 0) (status 10))
 (segment (start 140.081 86.741) (end 144.78 91.44) (width 0.25) (layer F.Cu) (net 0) (status 20))
 (segment (start 140.081 75.7028) (end 140.081 86.741) (width 0.25) (layer F.Cu) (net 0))
 (segment (start 140.0502 75.672) (end 140.081 75.7028) (width 0.25) (layer F.Cu) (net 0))
 (segment (start 138.29 75.172) (end 140.601 75.172) (width 0.25) (layer F.Cu) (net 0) (status 10))
 (segment (start 140.6144 84.7344) (end 144.78 88.9) (width 0.25) (layer F.Cu) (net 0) (status 20))
 (segment (start 140.6144 75.1854) (end 140.6144 84.7344) (width 0.25) (layer F.Cu) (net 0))
 (segment (start 140.601 75.172) (end 140.6144 75.1854) (width 0.25) (layer F.Cu) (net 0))
 (segment (start 138.29 74.672) (end 141.0248 74.672) (width 0.25) (layer F.Cu) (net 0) (status 10))
 (segment (start 141.1224 82.7024) (end 144.78 86.36) (width 0.25) (layer F.Cu) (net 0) (status 20))
 (segment (start 141.1224 74.7696) (end 141.1224 82.7024) (width 0.25) (layer F.Cu) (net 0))
 (segment (start 141.0248 74.672) (end 141.1224 74.7696) (width 0.25) (layer F.Cu) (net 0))
 (segment (start 138.29 74.172) (end 141.4566 74.172) (width 0.25) (layer F.Cu) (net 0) (status 10))
 (segment (start 141.605 80.645) (end 144.78 83.82) (width 0.25) (layer F.Cu) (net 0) (status 20))
 (segment (start 141.605 74.3204) (end 141.605 80.645) (width 0.25) (layer F.Cu) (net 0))
 (segment (start 141.4566 74.172) (end 141.605 74.3204) (width 0.25) (layer F.Cu) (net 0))
 (segment (start 138.29 73.672) (end 142.0996 73.672) (width 0.25) (layer F.Cu) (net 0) (status 10))
 (segment (start 142.113 78.613) (end 144.78 81.28) (width 0.25) (layer F.Cu) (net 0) (status 20))
 (segment (start 142.113 73.6854) (end 142.113 78.613) (width 0.25) (layer F.Cu) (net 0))
 (segment (start 142.0996 73.672) (end 142.113 73.6854) (width 0.25) (layer F.Cu) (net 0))
 (segment (start 138.29 73.172) (end 142.387 73.172) (width 0.25) (layer F.Cu) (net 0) (status 10))
 (segment (start 142.5702 76.5302) (end 144.78 78.74) (width 0.25) (layer F.Cu) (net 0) (status 20))
 (segment (start 142.5702 73.3552) (end 142.5702 76.5302) (width 0.25) (layer F.Cu) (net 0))
 (segment (start 142.387 73.172) (end 142.5702 73.3552) (width 0.25) (layer F.Cu) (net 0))
 (segment (start 138.29 72.672) (end 142.6744 72.672) (width 0.25) (layer F.Cu) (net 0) (status 10))
 (segment (start 143.1036 74.5236) (end 144.78 76.2) (width 0.25) (layer F.Cu) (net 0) (status 20))
 (segment (start 143.1036 73.1012) (end 143.1036 74.5236) (width 0.25) (layer F.Cu) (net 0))
 (segment (start 142.6744 72.672) (end 143.1036 73.1012) (width 0.25) (layer F.Cu) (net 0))
 (segment (start 134.14 72.022) (end 134.14 62.3036) (width 0.25) (layer F.Cu) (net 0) (status 10))
 (segment (start 140.5636 55.88) (end 144.78 55.88) (width 0.25) (layer F.Cu) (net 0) (status 20))
 (segment (start 134.14 62.3036) (end 140.5636 55.88) (width 0.25) (layer F.Cu) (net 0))
 (segment (start 134.64 72.022) (end 134.64 62.9212) (width 0.25) (layer F.Cu) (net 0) (status 10))
 (segment (start 139.1412 58.42) (end 144.78 58.42) (width 0.25) (layer F.Cu) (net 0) (status 20))
 (segment (start 134.64 62.9212) (end 139.1412 58.42) (width 0.25) (layer F.Cu) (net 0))
 (segment (start 144.1196 60.96) (end 144.78 60.96) (width 0.25) (layer F.Cu) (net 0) (status 30))
 (segment (start 137.14 72.022) (end 137.14 71.0638) (width 0.25) (layer F.Cu) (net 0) (status 10))
 (segment (start 137.3378 70.866) (end 144.526 70.866) (width 0.25) (layer F.Cu) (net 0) (status 20))
 (segment (start 137.14 71.0638) (end 137.3378 70.866) (width 0.25) (layer F.Cu) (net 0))
 (segment (start 144.526 70.866) (end 144.78 71.12) (width 0.25) (layer F.Cu) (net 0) (status 30))
 (segment (start 137.64 72.022) (end 143.142 72.022) (width 0.25) (layer F.Cu) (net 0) (status 10))
 (segment (start 143.142 72.022) (end 144.78 73.66) (width 0.25) (layer F.Cu) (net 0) (status 20))
 (segment (start 137.64 76.822) (end 137.64 83.34) (width 0.25) (layer F.Cu) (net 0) (status 10))
 (segment (start 137.64 83.34) (end 127 93.98) (width 0.25) (layer F.Cu) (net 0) (status 20))
 (segment (start 137.14 76.822) (end 137.14 81.3) (width 0.25) (layer F.Cu) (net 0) (status 10))
 (segment (start 137.14 81.3) (end 127 91.44) (width 0.25) (layer F.Cu) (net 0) (status 20))
 (segment (start 136.64 76.822) (end 136.64 79.133) (width 0.25) (layer F.Cu) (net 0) (status 10))
 (segment (start 136.64 79.133) (end 127 88.773) (width 0.25) (layer F.Cu) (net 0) (status 20))
 (segment (start 127 88.773) (end 127 88.9) (width 0.25) (layer F.Cu) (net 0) (status 30))
 (segment (start 136.14 76.822) (end 136.14 78.6932) (width 0.25) (layer F.Cu) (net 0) (status 10))
 (segment (start 128.4732 86.36) (end 127 86.36) (width 0.25) (layer F.Cu) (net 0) (status 20))
 (segment (start 136.14 78.6932) (end 128.4732 86.36) (width 0.25) (layer F.Cu) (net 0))
 (segment (start 135.64 76.822) (end 135.64 78.2788) (width 0.25) (layer F.Cu) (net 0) (status 10))
 (segment (start 130.0988 83.82) (end 127 83.82) (width 0.25) (layer F.Cu) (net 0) (status 20))
 (segment (start 135.64 78.2788) (end 130.0988 83.82) (width 0.25) (layer F.Cu) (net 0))
 (segment (start 135.14 76.822) (end 135.14 77.8644) (width 0.25) (layer F.Cu) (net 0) (status 10))
 (segment (start 131.7244 81.28) (end 127 81.28) (width 0.25) (layer F.Cu) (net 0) (status 20))
 (segment (start 135.14 77.8644) (end 131.7244 81.28) (width 0.25) (layer F.Cu) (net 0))
 (segment (start 134.64 76.822) (end 134.64 77.6932) (width 0.25) (layer F.Cu) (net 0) (status 10))
 (segment (start 133.5932 78.74) (end 127 78.74) (width 0.25) (layer F.Cu) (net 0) (status 20))
 (segment (start 134.64 77.6932) (end 133.5932 78.74) (width 0.25) (layer F.Cu) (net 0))
 (segment (start 134.14 76.822) (end 127.622 76.822) (width 0.25) (layer F.Cu) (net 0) (status 10))
 (segment (start 127.622 76.822) (end 127 76.2) (width 0.25) (layer F.Cu) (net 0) (status 20))
 (segment (start 133.49 76.172) (end 129.512 76.172) (width 0.25) (layer F.Cu) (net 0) (status 10))
 (segment (start 129.512 76.172) (end 127 73.66) (width 0.25) (layer F.Cu) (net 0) (status 20))
 (segment (start 133.49 75.672) (end 129.7994 75.672) (width 0.25) (layer F.Cu) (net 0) (status 10))
 (segment (start 129.3368 73.4568) (end 127 71.12) (width 0.25) (layer F.Cu) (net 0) (status 20))
 (segment (start 129.3368 75.2094) (end 129.3368 73.4568) (width 0.25) (layer F.Cu) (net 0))
 (segment (start 129.7994 75.672) (end 129.3368 75.2094) (width 0.25) (layer F.Cu) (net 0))
 (segment (start 133.49 75.172) (end 130.1108 75.172) (width 0.25) (layer F.Cu) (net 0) (status 10))
 (segment (start 129.8956 71.4756) (end 127 68.58) (width 0.25) (layer F.Cu) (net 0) (status 20))
 (segment (start 129.8956 74.9568) (end 129.8956 71.4756) (width 0.25) (layer F.Cu) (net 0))
 (segment (start 130.1108 75.172) (end 129.8956 74.9568) (width 0.25) (layer F.Cu) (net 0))
 (segment (start 133.49 74.672) (end 130.9076 74.672) (width 0.25) (layer F.Cu) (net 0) (status 10))
 (segment (start 130.4798 69.5198) (end 127 66.04) (width 0.25) (layer F.Cu) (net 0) (status 20))
 (segment (start 130.4798 74.2442) (end 130.4798 69.5198) (width 0.25) (layer F.Cu) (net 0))
 (segment (start 130.9076 74.672) (end 130.4798 74.2442) (width 0.25) (layer F.Cu) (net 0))
 (segment (start 133.49 74.172) (end 131.322 74.172) (width 0.25) (layer F.Cu) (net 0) (status 10))
 (segment (start 131.064 67.564) (end 127 63.5) (width 0.25) (layer F.Cu) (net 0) (status 20))
 (segment (start 131.064 73.914) (end 131.064 67.564) (width 0.25) (layer F.Cu) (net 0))
 (segment (start 131.322 74.172) (end 131.064 73.914) (width 0.25) (layer F.Cu) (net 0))
 (segment (start 133.49 73.672) (end 131.7872 73.672) (width 0.25) (layer F.Cu) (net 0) (status 10))
 (segment (start 131.6228 65.5828) (end 127 60.96) (width 0.25) (layer F.Cu) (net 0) (status 20))
 (segment (start 131.6228 73.5076) (end 131.6228 65.5828) (width 0.25) (layer F.Cu) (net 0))
 (segment (start 131.7872 73.672) (end 131.6228 73.5076) (width 0.25) (layer F.Cu) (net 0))
 (segment (start 133.49 73.172) (end 132.2778 73.172) (width 0.25) (layer F.Cu) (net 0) (status 10))
 (segment (start 132.1308 63.5508) (end 127 58.42) (width 0.25) (layer F.Cu) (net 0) (status 20))
 (segment (start 132.1308 73.025) (end 132.1308 63.5508) (width 0.25) (layer F.Cu) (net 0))
 (segment (start 132.2778 73.172) (end 132.1308 73.025) (width 0.25) (layer F.Cu) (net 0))
 (segment (start 133.49 72.672) (end 132.7684 72.672) (width 0.25) (layer F.Cu) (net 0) (status 10))
 (segment (start 132.6896 61.5696) (end 127 55.88) (width 0.25) (layer F.Cu) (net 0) (status 20))
 (segment (start 132.6896 72.5932) (end 132.6896 61.5696) (width 0.25) (layer F.Cu) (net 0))
 (segment (start 132.7684 72.672) (end 132.6896 72.5932) (width 0.25) (layer F.Cu) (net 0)))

